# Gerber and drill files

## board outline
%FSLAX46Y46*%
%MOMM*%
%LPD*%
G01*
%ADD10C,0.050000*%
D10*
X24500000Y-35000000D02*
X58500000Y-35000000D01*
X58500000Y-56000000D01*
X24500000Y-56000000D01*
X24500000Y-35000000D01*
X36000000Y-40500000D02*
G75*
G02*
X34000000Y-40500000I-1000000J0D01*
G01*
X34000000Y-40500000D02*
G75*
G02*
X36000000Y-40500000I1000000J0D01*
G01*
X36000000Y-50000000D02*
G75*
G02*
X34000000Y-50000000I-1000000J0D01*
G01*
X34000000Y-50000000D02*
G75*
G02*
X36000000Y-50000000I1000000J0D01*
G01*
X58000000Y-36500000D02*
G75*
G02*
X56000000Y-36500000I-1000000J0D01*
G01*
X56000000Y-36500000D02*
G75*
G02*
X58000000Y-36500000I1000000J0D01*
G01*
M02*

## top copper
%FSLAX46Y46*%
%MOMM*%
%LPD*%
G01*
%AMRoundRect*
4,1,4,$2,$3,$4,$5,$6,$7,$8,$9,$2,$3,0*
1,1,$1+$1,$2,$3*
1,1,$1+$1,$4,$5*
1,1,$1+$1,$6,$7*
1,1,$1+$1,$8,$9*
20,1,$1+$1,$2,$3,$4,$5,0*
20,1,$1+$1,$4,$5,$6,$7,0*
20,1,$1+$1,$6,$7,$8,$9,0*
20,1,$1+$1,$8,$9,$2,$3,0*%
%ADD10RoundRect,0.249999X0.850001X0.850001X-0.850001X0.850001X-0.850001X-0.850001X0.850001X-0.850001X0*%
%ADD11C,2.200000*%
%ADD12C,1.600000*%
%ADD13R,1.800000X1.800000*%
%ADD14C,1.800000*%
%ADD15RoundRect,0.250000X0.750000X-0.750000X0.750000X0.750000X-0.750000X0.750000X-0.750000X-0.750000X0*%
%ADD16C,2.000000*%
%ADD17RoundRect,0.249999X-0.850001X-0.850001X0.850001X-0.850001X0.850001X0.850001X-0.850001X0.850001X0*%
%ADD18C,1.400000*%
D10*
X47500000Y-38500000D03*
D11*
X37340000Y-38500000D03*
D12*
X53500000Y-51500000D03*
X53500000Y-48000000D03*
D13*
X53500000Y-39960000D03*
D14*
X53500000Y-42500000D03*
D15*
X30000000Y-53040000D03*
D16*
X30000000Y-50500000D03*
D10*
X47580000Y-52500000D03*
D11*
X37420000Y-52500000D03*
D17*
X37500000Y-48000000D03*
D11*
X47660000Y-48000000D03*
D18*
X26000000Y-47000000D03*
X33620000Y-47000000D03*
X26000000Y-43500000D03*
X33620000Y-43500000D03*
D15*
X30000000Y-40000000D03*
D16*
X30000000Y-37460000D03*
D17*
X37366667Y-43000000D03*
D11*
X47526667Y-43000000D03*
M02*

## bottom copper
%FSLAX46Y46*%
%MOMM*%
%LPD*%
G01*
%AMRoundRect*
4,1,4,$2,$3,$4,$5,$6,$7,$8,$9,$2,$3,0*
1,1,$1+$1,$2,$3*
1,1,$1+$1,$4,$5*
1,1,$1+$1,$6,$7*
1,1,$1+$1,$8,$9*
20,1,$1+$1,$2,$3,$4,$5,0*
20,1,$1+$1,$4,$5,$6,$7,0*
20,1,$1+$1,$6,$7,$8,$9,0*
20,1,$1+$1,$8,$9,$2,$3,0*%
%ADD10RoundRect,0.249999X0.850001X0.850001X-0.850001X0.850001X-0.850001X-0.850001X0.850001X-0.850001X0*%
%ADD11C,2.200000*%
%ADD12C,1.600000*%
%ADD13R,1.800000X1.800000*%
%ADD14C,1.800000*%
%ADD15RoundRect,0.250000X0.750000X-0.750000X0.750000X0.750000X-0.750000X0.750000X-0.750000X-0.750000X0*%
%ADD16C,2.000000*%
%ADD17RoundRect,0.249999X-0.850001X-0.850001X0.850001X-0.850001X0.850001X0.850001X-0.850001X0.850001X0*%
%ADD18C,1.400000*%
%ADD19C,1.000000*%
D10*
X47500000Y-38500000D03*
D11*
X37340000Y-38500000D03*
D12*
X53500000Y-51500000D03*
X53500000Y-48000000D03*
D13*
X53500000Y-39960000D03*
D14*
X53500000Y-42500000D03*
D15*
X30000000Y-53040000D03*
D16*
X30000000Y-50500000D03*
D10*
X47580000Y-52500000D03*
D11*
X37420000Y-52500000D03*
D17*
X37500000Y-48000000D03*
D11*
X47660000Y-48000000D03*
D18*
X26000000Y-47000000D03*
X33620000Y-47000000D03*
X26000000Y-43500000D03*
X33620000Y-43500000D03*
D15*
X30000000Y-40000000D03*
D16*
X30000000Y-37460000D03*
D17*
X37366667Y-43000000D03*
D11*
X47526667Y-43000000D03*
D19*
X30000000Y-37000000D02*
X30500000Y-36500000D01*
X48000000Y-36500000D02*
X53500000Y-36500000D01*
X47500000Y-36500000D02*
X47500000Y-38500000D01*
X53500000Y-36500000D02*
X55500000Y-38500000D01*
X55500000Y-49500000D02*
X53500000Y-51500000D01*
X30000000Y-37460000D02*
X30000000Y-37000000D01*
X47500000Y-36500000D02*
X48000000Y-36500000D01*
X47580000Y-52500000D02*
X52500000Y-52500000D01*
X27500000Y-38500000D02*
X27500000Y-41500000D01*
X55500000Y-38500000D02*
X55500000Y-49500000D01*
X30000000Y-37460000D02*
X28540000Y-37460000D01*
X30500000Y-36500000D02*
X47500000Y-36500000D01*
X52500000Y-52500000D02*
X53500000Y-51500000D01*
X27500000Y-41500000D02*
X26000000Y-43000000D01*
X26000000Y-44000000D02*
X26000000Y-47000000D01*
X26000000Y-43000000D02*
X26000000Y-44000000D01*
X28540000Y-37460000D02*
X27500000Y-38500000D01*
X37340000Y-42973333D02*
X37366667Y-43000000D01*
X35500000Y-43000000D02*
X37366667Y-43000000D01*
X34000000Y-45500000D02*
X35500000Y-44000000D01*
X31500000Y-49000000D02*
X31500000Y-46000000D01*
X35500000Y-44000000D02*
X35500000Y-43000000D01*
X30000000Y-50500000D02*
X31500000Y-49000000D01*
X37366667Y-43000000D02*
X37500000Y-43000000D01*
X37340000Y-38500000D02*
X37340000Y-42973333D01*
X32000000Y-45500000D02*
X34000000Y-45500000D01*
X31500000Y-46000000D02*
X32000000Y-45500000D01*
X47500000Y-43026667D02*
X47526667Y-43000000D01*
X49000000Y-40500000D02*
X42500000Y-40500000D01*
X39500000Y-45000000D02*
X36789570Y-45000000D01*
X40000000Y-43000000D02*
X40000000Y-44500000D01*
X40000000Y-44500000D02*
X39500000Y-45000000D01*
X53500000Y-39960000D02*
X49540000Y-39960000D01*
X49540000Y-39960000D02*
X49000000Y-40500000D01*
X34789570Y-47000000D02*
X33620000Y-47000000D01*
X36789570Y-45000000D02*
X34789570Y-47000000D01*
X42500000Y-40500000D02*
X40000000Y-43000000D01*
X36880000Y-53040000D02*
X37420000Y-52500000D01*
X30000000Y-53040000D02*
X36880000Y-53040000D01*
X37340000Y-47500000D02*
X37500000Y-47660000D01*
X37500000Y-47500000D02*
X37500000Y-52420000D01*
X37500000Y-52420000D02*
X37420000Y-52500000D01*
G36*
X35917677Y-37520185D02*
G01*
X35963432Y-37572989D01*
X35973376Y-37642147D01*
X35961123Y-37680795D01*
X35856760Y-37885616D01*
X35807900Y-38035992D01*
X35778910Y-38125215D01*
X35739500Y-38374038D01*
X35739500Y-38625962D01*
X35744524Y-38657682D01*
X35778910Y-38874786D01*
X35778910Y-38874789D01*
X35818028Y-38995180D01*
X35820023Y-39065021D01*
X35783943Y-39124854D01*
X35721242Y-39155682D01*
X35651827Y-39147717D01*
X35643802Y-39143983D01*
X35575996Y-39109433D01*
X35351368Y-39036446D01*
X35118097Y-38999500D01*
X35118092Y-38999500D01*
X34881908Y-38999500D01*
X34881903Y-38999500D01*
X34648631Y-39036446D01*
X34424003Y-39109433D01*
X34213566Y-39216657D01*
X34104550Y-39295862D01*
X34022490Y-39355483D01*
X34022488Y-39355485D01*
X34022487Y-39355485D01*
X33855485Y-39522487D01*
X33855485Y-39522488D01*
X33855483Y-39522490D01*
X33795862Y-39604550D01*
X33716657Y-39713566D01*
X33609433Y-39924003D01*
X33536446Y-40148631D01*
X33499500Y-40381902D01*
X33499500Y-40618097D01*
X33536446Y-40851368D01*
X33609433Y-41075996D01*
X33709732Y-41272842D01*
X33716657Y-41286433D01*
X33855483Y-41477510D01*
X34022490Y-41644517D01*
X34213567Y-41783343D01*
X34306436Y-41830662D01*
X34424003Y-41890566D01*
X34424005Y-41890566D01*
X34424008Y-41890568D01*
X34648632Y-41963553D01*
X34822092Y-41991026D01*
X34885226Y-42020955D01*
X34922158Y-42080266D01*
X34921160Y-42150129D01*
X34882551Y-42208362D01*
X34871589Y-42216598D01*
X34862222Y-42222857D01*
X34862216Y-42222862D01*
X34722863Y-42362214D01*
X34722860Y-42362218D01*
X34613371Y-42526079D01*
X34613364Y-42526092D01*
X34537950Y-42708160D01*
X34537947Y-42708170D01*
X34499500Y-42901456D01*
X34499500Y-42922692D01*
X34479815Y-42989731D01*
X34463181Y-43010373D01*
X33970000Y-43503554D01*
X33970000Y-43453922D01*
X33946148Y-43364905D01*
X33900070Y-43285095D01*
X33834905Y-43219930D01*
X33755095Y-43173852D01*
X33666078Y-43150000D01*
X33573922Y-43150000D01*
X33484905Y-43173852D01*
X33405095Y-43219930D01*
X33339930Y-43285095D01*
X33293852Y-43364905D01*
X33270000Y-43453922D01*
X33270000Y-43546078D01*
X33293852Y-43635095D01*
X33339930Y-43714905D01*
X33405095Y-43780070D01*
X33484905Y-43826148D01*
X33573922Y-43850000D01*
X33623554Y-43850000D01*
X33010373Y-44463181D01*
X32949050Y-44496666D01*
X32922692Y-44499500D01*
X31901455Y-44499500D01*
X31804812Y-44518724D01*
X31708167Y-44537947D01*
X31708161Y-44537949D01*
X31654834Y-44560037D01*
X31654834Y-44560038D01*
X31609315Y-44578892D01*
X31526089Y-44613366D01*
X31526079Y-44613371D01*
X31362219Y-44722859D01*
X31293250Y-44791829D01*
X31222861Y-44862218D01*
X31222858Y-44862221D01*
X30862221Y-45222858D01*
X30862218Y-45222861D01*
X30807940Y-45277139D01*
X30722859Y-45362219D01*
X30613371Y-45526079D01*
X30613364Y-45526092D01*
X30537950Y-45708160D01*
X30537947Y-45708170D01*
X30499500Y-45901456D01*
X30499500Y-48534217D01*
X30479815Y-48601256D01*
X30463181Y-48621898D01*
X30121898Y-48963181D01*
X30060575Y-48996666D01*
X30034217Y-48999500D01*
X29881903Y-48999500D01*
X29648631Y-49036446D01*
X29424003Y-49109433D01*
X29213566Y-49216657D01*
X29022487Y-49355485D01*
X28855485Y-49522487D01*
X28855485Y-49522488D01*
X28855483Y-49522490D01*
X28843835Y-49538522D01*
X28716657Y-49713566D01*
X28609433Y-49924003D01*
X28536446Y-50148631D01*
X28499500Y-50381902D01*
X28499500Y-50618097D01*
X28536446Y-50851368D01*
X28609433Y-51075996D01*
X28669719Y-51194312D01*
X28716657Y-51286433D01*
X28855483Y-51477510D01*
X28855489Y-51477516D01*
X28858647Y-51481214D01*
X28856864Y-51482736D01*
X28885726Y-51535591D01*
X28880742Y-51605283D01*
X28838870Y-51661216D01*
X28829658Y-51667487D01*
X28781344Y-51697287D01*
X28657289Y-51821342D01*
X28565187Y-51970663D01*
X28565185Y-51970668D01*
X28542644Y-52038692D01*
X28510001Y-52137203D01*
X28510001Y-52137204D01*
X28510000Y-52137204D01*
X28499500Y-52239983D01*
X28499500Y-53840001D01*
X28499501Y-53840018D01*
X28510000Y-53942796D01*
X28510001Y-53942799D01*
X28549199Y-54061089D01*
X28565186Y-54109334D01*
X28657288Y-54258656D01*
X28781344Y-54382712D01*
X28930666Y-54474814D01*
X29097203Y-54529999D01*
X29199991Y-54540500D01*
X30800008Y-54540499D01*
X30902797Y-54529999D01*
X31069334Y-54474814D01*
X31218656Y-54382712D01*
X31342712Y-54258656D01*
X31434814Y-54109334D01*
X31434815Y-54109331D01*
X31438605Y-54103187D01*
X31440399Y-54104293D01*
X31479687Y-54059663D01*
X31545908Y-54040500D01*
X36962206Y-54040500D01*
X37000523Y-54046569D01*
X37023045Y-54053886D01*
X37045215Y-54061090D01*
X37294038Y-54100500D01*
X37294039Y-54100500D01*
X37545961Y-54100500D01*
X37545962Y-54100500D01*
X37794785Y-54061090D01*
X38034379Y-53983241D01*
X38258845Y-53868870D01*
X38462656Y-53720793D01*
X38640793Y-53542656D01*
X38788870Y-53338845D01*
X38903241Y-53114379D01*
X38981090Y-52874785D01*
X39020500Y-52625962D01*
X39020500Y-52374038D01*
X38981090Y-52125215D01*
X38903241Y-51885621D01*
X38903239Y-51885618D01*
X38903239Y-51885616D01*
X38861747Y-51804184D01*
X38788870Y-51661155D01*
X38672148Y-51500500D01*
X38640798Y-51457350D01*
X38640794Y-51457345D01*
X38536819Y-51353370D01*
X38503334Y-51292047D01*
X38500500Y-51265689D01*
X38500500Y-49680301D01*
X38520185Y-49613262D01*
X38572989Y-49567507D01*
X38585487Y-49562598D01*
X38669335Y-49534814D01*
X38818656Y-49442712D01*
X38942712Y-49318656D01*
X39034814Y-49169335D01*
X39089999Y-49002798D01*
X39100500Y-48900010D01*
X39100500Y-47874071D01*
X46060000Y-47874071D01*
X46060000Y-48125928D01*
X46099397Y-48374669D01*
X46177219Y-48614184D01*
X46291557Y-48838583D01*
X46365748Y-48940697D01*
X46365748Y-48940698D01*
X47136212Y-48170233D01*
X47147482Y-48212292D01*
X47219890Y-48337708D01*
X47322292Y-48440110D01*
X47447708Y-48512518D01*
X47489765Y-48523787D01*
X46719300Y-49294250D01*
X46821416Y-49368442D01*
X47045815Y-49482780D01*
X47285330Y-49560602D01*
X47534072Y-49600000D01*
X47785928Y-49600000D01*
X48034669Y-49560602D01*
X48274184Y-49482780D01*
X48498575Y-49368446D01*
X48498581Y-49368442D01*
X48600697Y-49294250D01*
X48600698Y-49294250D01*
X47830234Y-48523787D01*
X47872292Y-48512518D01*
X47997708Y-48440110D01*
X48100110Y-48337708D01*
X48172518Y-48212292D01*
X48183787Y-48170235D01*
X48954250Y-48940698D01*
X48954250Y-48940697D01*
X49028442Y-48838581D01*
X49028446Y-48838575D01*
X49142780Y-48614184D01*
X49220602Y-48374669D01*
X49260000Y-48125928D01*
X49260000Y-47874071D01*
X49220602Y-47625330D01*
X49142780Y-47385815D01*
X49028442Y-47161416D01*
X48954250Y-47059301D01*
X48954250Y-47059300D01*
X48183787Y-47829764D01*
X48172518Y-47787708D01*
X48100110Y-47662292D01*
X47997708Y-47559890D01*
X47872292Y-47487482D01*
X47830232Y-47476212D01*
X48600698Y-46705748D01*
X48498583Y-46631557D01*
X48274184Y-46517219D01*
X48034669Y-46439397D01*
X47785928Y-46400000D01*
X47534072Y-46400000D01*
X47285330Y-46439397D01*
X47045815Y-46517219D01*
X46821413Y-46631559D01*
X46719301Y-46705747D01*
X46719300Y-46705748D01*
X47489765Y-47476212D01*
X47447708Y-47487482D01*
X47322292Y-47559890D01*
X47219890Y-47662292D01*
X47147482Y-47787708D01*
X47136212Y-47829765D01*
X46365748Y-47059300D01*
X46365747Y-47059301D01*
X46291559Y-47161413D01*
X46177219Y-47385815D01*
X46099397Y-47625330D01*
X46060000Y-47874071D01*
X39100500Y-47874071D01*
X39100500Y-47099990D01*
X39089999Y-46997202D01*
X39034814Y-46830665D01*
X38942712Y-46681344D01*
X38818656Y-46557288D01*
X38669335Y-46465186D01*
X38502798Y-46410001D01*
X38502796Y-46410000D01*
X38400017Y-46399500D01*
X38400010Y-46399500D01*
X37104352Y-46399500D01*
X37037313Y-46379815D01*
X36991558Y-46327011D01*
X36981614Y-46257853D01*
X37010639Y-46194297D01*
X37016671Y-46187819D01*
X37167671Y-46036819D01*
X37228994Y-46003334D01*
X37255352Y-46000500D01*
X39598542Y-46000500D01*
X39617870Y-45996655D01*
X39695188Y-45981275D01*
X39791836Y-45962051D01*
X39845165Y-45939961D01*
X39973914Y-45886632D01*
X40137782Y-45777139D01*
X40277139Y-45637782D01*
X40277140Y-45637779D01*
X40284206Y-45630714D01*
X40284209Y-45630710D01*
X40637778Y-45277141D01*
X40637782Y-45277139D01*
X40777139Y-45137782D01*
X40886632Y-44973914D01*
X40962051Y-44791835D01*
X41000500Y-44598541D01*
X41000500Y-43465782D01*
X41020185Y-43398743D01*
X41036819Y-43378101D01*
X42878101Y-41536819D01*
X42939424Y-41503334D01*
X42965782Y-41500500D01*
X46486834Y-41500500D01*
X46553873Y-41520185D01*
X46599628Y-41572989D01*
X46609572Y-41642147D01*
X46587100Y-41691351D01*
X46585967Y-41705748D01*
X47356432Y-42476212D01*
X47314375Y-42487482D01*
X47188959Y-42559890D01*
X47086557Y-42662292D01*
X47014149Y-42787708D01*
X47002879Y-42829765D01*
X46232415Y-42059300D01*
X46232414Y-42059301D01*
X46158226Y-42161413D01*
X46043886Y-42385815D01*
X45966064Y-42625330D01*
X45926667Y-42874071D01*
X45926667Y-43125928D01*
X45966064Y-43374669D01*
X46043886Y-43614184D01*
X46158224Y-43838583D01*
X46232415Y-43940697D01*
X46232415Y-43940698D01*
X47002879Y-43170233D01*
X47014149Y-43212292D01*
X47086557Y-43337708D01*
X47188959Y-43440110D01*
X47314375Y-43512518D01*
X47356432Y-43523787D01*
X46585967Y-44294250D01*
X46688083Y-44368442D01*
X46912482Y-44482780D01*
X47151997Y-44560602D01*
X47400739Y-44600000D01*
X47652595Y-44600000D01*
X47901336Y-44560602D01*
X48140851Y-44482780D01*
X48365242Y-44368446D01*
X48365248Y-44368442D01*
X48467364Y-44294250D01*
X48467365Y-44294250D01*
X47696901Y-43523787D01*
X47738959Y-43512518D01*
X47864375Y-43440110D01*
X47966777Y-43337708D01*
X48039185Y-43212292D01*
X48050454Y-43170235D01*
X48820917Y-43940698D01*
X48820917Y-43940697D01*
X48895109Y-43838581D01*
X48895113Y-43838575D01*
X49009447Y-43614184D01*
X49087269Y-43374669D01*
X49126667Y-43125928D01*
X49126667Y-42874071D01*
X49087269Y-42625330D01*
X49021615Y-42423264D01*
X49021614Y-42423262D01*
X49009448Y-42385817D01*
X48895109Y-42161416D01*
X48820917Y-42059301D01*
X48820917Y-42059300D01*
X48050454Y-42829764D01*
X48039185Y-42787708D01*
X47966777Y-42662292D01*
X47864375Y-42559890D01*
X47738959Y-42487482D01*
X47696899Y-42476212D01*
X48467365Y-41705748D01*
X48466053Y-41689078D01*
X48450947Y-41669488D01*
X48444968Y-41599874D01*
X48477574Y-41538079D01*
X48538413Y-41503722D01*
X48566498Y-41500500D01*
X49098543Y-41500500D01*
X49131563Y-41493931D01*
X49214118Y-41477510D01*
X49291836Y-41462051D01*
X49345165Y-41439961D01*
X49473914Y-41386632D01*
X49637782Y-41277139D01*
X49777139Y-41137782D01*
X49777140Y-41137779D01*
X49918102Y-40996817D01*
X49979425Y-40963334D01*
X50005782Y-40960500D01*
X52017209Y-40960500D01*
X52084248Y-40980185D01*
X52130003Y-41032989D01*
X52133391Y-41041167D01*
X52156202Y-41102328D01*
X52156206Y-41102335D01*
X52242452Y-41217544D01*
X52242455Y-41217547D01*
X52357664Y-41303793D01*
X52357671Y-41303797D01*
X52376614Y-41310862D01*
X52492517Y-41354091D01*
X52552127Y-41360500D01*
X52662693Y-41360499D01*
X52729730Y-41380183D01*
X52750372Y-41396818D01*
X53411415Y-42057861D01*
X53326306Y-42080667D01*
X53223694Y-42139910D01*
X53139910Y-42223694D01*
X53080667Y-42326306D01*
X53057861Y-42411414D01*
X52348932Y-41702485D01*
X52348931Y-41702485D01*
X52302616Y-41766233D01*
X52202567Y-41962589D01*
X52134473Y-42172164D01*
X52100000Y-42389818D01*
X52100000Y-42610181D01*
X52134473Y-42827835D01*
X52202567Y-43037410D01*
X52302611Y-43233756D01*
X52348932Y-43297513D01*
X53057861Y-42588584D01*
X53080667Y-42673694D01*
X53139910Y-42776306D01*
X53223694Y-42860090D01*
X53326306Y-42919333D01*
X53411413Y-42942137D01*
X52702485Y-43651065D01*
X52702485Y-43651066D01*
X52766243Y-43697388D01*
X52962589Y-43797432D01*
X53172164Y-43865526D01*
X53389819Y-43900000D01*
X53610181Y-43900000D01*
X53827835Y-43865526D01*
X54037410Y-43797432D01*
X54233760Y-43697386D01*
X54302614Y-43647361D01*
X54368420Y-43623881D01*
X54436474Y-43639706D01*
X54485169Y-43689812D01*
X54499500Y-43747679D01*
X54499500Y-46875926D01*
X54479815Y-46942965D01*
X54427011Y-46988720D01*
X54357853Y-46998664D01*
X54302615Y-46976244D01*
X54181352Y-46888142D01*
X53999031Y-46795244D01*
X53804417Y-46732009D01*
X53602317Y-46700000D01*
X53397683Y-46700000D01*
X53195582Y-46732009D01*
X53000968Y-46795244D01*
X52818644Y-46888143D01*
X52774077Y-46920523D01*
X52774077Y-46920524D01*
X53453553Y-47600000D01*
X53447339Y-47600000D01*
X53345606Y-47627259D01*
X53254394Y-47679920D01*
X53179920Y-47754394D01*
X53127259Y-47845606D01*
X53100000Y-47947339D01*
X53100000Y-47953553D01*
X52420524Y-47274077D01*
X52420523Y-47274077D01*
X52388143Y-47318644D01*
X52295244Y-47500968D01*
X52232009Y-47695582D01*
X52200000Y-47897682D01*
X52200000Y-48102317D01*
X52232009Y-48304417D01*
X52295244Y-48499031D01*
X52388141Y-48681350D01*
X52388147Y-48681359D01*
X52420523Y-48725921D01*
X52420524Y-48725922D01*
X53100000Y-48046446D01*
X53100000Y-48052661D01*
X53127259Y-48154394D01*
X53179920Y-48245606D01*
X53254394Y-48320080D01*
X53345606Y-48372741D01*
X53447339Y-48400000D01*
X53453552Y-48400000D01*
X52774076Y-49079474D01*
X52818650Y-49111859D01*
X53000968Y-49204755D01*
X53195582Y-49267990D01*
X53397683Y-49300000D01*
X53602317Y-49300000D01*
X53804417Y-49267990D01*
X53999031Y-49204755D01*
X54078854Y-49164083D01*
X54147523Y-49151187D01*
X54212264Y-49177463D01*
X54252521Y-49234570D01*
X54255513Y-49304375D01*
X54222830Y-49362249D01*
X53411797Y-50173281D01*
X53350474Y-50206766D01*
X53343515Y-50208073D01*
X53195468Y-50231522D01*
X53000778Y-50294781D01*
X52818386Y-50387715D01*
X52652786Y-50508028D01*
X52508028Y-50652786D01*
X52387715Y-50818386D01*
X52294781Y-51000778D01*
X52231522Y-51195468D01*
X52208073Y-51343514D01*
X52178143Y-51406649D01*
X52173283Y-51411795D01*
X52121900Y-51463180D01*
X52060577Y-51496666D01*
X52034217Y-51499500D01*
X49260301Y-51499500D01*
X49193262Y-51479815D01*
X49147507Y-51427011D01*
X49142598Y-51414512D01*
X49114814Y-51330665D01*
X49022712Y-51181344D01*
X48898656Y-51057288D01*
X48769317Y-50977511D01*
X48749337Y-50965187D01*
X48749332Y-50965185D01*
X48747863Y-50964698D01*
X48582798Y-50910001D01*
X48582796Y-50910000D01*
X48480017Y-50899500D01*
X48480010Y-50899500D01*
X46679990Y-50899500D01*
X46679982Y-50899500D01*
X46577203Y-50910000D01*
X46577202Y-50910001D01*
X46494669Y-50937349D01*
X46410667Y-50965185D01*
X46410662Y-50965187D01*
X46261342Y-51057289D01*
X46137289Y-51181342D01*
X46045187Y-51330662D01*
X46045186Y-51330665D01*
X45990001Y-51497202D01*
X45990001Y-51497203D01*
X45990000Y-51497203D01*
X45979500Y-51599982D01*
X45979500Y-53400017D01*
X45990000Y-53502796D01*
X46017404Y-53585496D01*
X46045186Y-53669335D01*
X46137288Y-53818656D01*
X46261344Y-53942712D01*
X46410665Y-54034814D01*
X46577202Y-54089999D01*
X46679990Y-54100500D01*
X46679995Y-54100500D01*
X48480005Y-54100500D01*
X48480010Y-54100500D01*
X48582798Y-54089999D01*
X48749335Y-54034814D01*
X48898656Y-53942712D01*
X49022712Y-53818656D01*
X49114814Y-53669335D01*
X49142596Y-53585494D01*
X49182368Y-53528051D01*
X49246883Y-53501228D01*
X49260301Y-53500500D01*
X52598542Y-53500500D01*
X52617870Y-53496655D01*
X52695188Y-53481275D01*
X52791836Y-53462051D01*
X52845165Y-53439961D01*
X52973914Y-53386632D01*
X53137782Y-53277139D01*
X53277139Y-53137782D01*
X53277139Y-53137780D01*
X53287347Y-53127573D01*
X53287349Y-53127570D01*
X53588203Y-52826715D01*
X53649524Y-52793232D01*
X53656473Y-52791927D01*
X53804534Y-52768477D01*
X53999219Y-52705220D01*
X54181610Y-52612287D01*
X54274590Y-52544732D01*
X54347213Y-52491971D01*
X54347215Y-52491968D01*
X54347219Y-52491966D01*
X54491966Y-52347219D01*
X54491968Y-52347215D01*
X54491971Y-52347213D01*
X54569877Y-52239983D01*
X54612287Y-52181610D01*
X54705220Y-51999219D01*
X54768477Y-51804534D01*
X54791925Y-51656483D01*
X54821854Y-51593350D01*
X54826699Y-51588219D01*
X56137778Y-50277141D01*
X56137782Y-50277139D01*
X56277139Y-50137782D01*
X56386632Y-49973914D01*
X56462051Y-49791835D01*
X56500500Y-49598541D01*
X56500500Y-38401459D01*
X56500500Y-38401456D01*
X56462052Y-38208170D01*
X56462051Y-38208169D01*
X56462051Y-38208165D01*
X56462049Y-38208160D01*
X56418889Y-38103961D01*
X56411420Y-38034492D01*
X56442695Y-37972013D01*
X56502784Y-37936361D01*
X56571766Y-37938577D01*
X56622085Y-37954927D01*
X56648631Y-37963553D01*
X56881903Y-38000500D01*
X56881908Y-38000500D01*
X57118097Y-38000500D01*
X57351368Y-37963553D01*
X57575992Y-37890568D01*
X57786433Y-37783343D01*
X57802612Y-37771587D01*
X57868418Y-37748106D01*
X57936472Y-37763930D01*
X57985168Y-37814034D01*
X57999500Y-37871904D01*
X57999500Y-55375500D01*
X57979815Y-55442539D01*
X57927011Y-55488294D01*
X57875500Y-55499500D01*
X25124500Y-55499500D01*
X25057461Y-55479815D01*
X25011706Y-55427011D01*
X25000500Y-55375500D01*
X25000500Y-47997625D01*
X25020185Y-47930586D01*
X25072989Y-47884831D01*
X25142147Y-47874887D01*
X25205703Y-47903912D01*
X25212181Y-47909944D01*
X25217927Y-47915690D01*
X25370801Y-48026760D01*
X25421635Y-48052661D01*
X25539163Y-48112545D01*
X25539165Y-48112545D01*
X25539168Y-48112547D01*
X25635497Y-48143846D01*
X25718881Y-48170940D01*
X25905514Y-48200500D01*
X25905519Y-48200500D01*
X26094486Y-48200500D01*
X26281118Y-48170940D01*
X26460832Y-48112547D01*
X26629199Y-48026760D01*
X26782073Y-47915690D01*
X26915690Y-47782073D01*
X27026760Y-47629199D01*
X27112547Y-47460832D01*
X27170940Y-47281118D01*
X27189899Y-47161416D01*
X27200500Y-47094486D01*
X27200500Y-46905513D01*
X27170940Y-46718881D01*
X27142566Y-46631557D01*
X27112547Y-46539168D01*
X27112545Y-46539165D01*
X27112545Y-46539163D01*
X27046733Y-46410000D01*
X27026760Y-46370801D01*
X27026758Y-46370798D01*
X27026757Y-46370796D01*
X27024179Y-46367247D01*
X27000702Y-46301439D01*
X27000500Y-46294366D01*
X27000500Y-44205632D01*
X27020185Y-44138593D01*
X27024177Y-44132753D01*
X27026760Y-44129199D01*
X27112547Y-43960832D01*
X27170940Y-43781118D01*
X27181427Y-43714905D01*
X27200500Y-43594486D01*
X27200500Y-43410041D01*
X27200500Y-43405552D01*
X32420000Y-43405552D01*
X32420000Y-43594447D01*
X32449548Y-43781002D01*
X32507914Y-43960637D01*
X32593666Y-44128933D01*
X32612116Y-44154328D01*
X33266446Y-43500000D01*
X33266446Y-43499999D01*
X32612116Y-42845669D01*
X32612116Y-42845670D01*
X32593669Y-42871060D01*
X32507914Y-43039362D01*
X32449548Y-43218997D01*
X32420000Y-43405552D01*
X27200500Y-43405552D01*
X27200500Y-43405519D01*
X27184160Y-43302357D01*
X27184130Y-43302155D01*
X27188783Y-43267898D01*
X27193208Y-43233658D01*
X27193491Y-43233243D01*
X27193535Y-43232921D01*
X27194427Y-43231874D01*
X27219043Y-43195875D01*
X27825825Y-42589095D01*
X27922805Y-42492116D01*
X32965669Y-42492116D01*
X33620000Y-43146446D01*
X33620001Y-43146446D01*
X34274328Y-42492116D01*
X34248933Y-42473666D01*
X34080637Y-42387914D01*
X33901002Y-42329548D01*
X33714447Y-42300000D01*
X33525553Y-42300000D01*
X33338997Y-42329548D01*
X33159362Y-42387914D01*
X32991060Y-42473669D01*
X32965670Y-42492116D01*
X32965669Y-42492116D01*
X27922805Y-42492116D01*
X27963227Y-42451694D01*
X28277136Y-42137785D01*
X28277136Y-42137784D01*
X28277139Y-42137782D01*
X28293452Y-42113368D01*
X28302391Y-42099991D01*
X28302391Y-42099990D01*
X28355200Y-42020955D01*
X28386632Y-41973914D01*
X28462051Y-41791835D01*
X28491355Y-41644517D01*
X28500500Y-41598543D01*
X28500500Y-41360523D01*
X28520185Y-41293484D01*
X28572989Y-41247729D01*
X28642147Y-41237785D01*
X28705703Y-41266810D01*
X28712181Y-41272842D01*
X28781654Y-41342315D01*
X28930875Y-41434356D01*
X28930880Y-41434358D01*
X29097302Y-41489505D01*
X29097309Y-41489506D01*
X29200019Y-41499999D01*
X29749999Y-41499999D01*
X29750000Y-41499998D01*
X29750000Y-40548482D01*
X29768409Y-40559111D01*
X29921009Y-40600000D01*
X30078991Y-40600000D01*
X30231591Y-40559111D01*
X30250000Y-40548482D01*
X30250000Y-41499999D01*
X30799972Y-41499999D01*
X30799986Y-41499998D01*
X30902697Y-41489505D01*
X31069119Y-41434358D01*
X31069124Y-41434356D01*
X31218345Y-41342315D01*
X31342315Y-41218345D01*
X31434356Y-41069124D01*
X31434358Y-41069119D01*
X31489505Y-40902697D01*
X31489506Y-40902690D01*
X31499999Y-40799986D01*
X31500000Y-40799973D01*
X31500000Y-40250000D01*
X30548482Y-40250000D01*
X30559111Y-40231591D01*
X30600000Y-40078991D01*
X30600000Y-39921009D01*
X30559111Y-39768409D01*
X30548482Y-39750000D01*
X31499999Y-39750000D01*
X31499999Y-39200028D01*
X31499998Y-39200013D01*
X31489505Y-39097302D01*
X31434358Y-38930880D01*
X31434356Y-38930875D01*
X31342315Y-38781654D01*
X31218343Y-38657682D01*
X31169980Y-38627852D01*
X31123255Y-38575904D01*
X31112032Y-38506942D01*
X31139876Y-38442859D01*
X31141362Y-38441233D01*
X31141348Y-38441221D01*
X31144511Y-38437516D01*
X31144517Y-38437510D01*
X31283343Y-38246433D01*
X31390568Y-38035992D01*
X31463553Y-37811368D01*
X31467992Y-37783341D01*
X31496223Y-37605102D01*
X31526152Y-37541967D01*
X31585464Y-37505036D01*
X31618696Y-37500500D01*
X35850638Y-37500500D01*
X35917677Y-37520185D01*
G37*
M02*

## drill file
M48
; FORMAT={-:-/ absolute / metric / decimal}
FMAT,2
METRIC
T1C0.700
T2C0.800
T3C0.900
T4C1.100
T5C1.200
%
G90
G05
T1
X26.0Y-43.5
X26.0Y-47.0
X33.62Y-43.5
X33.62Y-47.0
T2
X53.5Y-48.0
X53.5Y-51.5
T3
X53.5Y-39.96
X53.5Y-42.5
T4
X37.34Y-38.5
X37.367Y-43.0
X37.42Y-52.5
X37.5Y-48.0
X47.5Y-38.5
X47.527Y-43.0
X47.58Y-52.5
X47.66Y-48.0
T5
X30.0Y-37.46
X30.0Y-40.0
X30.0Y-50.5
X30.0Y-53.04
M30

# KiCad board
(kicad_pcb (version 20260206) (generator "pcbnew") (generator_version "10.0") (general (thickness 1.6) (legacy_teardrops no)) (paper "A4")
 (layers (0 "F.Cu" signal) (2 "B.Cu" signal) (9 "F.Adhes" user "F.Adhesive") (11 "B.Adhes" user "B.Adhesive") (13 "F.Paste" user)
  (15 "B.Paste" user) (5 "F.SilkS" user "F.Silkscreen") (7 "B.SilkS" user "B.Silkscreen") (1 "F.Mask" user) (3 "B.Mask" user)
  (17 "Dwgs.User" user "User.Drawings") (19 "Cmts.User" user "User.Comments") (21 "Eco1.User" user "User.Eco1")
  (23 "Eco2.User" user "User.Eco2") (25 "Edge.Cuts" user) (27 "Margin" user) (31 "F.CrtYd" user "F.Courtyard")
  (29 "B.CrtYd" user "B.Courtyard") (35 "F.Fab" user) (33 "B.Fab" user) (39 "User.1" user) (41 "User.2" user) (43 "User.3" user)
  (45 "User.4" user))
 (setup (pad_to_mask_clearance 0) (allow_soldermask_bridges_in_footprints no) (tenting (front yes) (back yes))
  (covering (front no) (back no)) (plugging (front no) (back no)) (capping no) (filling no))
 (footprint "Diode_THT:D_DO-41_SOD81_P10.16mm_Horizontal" (layer "F.Cu") (at 47.5 38.5 180)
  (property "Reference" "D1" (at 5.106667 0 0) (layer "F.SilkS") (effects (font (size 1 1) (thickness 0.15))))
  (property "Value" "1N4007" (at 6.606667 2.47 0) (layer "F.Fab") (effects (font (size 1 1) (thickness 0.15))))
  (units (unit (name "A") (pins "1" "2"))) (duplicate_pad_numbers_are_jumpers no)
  (pad "1" thru_hole roundrect (at 0 0 180) (size 2.2 2.2) (drill 1.1) (layers "*.Cu" "*.Mask") (remove_unused_layers no)
   (roundrect_rratio 0.113636) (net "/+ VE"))
  (pad "2" thru_hole circle (at 10.16 0 180) (size 2.2 2.2) (drill 1.1) (layers "*.Cu" "*.Mask") (remove_unused_layers no)
   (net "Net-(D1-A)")))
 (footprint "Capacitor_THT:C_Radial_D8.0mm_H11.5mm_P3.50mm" (layer "F.Cu") (at 53.5 51.5 90)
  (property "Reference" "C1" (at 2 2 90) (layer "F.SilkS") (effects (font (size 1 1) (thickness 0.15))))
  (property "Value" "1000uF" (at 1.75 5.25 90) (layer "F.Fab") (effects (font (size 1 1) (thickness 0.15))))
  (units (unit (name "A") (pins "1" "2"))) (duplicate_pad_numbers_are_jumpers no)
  (pad "1" thru_hole circle (at 0 0 90) (size 1.6 1.6) (drill 0.8) (layers "*.Cu" "*.Mask") (remove_unused_layers no) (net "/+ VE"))
  (pad "2" thru_hole circle (at 3.5 0 90) (size 1.6 1.6) (drill 0.8) (layers "*.Cu" "*.Mask") (remove_unused_layers no) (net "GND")))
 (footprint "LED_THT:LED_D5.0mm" (layer "F.Cu") (at 53.5 39.96 -90)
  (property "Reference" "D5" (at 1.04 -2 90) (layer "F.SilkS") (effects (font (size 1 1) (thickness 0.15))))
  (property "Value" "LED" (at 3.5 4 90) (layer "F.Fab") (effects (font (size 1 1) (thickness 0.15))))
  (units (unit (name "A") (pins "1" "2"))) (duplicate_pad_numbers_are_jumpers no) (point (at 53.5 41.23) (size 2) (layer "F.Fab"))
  (pad "1" thru_hole rect (at 0 0 270) (size 1.8 1.8) (drill 0.9) (layers "*.Cu" "*.Mask") (remove_unused_layers no) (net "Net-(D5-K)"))
  (pad "2" thru_hole circle (at 2.54 0 270) (size 1.8 1.8) (drill 0.9) (layers "*.Cu" "*.Mask") (remove_unused_layers no) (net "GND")))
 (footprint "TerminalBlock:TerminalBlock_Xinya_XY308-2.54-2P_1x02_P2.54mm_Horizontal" (layer "F.Cu") (at 30 53.04 90)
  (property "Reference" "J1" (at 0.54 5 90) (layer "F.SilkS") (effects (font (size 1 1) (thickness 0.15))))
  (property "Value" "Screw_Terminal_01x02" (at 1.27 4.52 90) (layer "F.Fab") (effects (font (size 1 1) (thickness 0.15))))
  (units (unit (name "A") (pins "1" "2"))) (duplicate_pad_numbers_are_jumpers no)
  (pad "1" thru_hole roundrect (at 0 0 90) (size 2 2) (drill 1.2) (layers "*.Cu" "*.Mask") (remove_unused_layers no)
   (roundrect_rratio 0.125) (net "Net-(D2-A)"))
  (pad "2" thru_hole circle (at 2.54 0 90) (size 2 2) (drill 1.2) (layers "*.Cu" "*.Mask") (remove_unused_layers no) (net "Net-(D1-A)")))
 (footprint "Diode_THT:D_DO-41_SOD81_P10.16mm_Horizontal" (layer "F.Cu") (at 47.58 52.5 180)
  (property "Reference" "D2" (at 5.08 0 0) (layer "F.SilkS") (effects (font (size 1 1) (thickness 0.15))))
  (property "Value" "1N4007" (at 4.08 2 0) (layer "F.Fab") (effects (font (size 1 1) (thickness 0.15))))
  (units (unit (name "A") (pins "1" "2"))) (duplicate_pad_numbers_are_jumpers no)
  (pad "1" thru_hole roundrect (at 0 0 180) (size 2.2 2.2) (drill 1.1) (layers "*.Cu" "*.Mask") (remove_unused_layers no)
   (roundrect_rratio 0.113636) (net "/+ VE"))
  (pad "2" thru_hole circle (at 10.16 0 180) (size 2.2 2.2) (drill 1.1) (layers "*.Cu" "*.Mask") (remove_unused_layers no)
   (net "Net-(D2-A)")))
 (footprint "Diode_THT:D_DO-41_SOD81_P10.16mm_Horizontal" (layer "F.Cu") (at 37.5 48)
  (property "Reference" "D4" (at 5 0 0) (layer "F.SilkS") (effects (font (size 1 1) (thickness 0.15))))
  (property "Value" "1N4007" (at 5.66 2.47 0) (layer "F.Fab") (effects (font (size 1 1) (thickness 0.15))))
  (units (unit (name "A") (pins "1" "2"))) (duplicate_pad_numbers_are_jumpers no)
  (pad "1" thru_hole roundrect (at 0 0) (size 2.2 2.2) (drill 1.1) (layers "*.Cu" "*.Mask") (remove_unused_layers no)
   (roundrect_rratio 0.113636) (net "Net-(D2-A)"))
  (pad "2" thru_hole circle (at 10.16 0) (size 2.2 2.2) (drill 1.1) (layers "*.Cu" "*.Mask") (remove_unused_layers no) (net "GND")))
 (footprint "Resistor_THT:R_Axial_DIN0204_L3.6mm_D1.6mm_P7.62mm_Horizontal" (layer "F.Cu") (at 26 47)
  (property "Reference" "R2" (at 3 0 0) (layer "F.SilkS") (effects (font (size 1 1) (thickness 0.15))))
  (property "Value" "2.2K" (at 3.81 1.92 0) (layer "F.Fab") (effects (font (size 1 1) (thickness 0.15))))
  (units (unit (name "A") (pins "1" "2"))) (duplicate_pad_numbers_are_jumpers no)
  (pad "1" thru_hole circle (at 0 0) (size 1.4 1.4) (drill 0.7) (layers "*.Cu" "*.Mask") (remove_unused_layers no) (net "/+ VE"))
  (pad "2" thru_hole circle (at 7.62 0) (size 1.4 1.4) (drill 0.7) (layers "*.Cu" "*.Mask") (remove_unused_layers no) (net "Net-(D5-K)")))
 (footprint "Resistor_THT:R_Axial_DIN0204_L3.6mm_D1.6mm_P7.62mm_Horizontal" (layer "F.Cu") (at 26 43.5)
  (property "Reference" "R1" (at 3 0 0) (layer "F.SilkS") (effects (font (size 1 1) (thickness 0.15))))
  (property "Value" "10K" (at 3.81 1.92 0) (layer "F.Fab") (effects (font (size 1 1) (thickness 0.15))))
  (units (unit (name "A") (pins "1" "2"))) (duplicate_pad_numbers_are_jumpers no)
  (pad "1" thru_hole circle (at 0 0) (size 1.4 1.4) (drill 0.7) (layers "*.Cu" "*.Mask") (remove_unused_layers no) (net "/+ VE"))
  (pad "2" thru_hole circle (at 7.62 0) (size 1.4 1.4) (drill 0.7) (layers "*.Cu" "*.Mask") (remove_unused_layers no) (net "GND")))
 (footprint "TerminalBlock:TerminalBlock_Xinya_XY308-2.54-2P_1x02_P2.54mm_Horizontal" (layer "F.Cu") (at 30 40 90)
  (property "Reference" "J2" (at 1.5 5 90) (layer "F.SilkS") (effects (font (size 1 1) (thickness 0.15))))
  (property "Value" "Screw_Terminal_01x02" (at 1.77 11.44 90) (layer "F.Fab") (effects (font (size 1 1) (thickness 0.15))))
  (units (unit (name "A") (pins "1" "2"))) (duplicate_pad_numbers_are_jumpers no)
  (pad "1" thru_hole roundrect (at 0 0 90) (size 2 2) (drill 1.2) (layers "*.Cu" "*.Mask") (remove_unused_layers no)
   (roundrect_rratio 0.125) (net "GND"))
  (pad "2" thru_hole circle (at 2.54 0 90) (size 2 2) (drill 1.2) (layers "*.Cu" "*.Mask") (remove_unused_layers no) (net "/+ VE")))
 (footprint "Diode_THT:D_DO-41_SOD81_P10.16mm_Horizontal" (layer "F.Cu") (at 37.366667 43)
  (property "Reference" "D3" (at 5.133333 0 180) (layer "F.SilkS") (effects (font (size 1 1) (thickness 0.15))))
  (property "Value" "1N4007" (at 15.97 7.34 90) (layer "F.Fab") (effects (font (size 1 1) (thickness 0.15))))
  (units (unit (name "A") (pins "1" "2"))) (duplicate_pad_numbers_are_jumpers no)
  (pad "1" thru_hole roundrect (at 0 0) (size 2.2 2.2) (drill 1.1) (layers "*.Cu" "*.Mask") (remove_unused_layers no)
   (roundrect_rratio 0.113636) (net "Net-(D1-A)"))
  (pad "2" thru_hole circle (at 10.16 0) (size 2.2 2.2) (drill 1.1) (layers "*.Cu" "*.Mask") (remove_unused_layers no) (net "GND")))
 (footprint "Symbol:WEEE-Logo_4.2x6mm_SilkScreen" (layer "B.Cu") (at 43 52.5 180)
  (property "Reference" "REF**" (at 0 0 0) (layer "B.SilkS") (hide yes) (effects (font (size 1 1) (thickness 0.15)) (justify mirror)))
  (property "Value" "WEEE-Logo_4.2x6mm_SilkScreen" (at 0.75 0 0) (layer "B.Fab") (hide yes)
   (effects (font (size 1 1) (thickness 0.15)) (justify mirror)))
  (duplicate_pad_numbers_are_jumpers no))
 (gr_rect (start 24.5 35) (end 58.5 56) (stroke (width 0.05) (type default)) (fill no) (layer "Edge.Cuts"))
 (gr_circle (center 35 40.5) (end 34 40.5) (stroke (width 0.05) (type default)) (fill no) (layer "Edge.Cuts"))
 (gr_circle (center 35 50) (end 34 50) (stroke (width 0.05) (type default)) (fill no) (layer "Edge.Cuts"))
 (gr_circle (center 57 36.5) (end 56 36.5) (stroke (width 0.05) (type default)) (fill no) (layer "Edge.Cuts"))
 (segment (start 30 37) (end 30.5 36.5) (width 1) (layer "B.Cu") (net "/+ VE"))
 (segment (start 48 36.5) (end 53.5 36.5) (width 1) (layer "B.Cu") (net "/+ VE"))
 (segment (start 47.5 36.5) (end 47.5 38.5) (width 1) (layer "B.Cu") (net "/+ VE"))
 (segment (start 53.5 36.5) (end 55.5 38.5) (width 1) (layer "B.Cu") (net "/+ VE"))
 (segment (start 55.5 49.5) (end 53.5 51.5) (width 1) (layer "B.Cu") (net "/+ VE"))
 (segment (start 30 37.46) (end 30 37) (width 1) (layer "B.Cu") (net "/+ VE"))
 (segment (start 47.5 36.5) (end 48 36.5) (width 1) (layer "B.Cu") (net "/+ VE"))
 (segment (start 47.58 52.5) (end 52.5 52.5) (width 1) (layer "B.Cu") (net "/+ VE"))
 (segment (start 27.5 38.5) (end 27.5 41.5) (width 1) (layer "B.Cu") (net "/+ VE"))
 (segment (start 55.5 38.5) (end 55.5 49.5) (width 1) (layer "B.Cu") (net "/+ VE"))
 (segment (start 30 37.46) (end 28.54 37.46) (width 1) (layer "B.Cu") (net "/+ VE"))
 (segment (start 30.5 36.5) (end 47.5 36.5) (width 1) (layer "B.Cu") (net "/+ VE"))
 (segment (start 52.5 52.5) (end 53.5 51.5) (width 1) (layer "B.Cu") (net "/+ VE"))
 (segment (start 27.5 41.5) (end 26 43) (width 1) (layer "B.Cu") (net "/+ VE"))
 (segment (start 26 44) (end 26 47) (width 1) (layer "B.Cu") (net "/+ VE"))
 (segment (start 26 43) (end 26 44) (width 1) (layer "B.Cu") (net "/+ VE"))
 (segment (start 28.54 37.46) (end 27.5 38.5) (width 1) (layer "B.Cu") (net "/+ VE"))
 (segment (start 37.34 42.973333) (end 37.366667 43) (width 1) (layer "B.Cu") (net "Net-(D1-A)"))
 (segment (start 35.5 43) (end 37.366667 43) (width 1) (layer "B.Cu") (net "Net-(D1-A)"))
 (segment (start 34 45.5) (end 35.5 44) (width 1) (layer "B.Cu") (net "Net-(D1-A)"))
 (segment (start 31.5 49) (end 31.5 46) (width 1) (layer "B.Cu") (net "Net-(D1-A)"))
 (segment (start 35.5 44) (end 35.5 43) (width 1) (layer "B.Cu") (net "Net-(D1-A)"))
 (segment (start 30 50.5) (end 31.5 49) (width 1) (layer "B.Cu") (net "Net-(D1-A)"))
 (segment (start 37.366667 43) (end 37.5 43) (width 1) (layer "B.Cu") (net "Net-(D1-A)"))
 (segment (start 37.34 38.5) (end 37.34 42.973333) (width 1) (layer "B.Cu") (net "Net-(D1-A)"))
 (segment (start 32 45.5) (end 34 45.5) (width 1) (layer "B.Cu") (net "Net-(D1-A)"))
 (segment (start 31.5 46) (end 32 45.5) (width 1) (layer "B.Cu") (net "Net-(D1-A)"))
 (segment (start 47.5 43.026667) (end 47.526667 43) (width 1) (layer "B.Cu") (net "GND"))
 (segment (start 49 40.5) (end 42.5 40.5) (width 1) (layer "B.Cu") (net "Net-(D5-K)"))
 (segment (start 39.5 45) (end 36.78957 45) (width 1) (layer "B.Cu") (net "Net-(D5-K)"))
 (segment (start 40 43) (end 40 44.5) (width 1) (layer "B.Cu") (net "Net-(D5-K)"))
 (segment (start 40 44.5) (end 39.5 45) (width 1) (layer "B.Cu") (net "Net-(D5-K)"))
 (segment (start 53.5 39.96) (end 49.54 39.96) (width 1) (layer "B.Cu") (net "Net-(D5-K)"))
 (segment (start 49.54 39.96) (end 49 40.5) (width 1) (layer "B.Cu") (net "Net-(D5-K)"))
 (segment (start 34.78957 47) (end 33.62 47) (width 1) (layer "B.Cu") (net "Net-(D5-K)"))
 (segment (start 36.78957 45) (end 34.78957 47) (width 1) (layer "B.Cu") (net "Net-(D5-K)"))
 (segment (start 42.5 40.5) (end 40 43) (width 1) (layer "B.Cu") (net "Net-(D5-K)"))
 (segment (start 36.88 53.04) (end 37.42 52.5) (width 1) (layer "B.Cu") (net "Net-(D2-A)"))
 (segment (start 30 53.04) (end 36.88 53.04) (width 1) (layer "B.Cu") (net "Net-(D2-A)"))
 (segment (start 37.34 47.5) (end 37.5 47.66) (width 1) (layer "B.Cu") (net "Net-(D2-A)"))
 (segment (start 37.5 47.5) (end 37.5 52.42) (width 1) (layer "B.Cu") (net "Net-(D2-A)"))
 (segment (start 37.5 52.42) (end 37.42 52.5) (width 1) (layer "B.Cu") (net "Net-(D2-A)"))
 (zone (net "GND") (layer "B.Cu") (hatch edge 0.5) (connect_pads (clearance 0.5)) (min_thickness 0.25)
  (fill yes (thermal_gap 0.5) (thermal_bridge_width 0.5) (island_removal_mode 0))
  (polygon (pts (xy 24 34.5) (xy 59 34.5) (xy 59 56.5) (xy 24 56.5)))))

